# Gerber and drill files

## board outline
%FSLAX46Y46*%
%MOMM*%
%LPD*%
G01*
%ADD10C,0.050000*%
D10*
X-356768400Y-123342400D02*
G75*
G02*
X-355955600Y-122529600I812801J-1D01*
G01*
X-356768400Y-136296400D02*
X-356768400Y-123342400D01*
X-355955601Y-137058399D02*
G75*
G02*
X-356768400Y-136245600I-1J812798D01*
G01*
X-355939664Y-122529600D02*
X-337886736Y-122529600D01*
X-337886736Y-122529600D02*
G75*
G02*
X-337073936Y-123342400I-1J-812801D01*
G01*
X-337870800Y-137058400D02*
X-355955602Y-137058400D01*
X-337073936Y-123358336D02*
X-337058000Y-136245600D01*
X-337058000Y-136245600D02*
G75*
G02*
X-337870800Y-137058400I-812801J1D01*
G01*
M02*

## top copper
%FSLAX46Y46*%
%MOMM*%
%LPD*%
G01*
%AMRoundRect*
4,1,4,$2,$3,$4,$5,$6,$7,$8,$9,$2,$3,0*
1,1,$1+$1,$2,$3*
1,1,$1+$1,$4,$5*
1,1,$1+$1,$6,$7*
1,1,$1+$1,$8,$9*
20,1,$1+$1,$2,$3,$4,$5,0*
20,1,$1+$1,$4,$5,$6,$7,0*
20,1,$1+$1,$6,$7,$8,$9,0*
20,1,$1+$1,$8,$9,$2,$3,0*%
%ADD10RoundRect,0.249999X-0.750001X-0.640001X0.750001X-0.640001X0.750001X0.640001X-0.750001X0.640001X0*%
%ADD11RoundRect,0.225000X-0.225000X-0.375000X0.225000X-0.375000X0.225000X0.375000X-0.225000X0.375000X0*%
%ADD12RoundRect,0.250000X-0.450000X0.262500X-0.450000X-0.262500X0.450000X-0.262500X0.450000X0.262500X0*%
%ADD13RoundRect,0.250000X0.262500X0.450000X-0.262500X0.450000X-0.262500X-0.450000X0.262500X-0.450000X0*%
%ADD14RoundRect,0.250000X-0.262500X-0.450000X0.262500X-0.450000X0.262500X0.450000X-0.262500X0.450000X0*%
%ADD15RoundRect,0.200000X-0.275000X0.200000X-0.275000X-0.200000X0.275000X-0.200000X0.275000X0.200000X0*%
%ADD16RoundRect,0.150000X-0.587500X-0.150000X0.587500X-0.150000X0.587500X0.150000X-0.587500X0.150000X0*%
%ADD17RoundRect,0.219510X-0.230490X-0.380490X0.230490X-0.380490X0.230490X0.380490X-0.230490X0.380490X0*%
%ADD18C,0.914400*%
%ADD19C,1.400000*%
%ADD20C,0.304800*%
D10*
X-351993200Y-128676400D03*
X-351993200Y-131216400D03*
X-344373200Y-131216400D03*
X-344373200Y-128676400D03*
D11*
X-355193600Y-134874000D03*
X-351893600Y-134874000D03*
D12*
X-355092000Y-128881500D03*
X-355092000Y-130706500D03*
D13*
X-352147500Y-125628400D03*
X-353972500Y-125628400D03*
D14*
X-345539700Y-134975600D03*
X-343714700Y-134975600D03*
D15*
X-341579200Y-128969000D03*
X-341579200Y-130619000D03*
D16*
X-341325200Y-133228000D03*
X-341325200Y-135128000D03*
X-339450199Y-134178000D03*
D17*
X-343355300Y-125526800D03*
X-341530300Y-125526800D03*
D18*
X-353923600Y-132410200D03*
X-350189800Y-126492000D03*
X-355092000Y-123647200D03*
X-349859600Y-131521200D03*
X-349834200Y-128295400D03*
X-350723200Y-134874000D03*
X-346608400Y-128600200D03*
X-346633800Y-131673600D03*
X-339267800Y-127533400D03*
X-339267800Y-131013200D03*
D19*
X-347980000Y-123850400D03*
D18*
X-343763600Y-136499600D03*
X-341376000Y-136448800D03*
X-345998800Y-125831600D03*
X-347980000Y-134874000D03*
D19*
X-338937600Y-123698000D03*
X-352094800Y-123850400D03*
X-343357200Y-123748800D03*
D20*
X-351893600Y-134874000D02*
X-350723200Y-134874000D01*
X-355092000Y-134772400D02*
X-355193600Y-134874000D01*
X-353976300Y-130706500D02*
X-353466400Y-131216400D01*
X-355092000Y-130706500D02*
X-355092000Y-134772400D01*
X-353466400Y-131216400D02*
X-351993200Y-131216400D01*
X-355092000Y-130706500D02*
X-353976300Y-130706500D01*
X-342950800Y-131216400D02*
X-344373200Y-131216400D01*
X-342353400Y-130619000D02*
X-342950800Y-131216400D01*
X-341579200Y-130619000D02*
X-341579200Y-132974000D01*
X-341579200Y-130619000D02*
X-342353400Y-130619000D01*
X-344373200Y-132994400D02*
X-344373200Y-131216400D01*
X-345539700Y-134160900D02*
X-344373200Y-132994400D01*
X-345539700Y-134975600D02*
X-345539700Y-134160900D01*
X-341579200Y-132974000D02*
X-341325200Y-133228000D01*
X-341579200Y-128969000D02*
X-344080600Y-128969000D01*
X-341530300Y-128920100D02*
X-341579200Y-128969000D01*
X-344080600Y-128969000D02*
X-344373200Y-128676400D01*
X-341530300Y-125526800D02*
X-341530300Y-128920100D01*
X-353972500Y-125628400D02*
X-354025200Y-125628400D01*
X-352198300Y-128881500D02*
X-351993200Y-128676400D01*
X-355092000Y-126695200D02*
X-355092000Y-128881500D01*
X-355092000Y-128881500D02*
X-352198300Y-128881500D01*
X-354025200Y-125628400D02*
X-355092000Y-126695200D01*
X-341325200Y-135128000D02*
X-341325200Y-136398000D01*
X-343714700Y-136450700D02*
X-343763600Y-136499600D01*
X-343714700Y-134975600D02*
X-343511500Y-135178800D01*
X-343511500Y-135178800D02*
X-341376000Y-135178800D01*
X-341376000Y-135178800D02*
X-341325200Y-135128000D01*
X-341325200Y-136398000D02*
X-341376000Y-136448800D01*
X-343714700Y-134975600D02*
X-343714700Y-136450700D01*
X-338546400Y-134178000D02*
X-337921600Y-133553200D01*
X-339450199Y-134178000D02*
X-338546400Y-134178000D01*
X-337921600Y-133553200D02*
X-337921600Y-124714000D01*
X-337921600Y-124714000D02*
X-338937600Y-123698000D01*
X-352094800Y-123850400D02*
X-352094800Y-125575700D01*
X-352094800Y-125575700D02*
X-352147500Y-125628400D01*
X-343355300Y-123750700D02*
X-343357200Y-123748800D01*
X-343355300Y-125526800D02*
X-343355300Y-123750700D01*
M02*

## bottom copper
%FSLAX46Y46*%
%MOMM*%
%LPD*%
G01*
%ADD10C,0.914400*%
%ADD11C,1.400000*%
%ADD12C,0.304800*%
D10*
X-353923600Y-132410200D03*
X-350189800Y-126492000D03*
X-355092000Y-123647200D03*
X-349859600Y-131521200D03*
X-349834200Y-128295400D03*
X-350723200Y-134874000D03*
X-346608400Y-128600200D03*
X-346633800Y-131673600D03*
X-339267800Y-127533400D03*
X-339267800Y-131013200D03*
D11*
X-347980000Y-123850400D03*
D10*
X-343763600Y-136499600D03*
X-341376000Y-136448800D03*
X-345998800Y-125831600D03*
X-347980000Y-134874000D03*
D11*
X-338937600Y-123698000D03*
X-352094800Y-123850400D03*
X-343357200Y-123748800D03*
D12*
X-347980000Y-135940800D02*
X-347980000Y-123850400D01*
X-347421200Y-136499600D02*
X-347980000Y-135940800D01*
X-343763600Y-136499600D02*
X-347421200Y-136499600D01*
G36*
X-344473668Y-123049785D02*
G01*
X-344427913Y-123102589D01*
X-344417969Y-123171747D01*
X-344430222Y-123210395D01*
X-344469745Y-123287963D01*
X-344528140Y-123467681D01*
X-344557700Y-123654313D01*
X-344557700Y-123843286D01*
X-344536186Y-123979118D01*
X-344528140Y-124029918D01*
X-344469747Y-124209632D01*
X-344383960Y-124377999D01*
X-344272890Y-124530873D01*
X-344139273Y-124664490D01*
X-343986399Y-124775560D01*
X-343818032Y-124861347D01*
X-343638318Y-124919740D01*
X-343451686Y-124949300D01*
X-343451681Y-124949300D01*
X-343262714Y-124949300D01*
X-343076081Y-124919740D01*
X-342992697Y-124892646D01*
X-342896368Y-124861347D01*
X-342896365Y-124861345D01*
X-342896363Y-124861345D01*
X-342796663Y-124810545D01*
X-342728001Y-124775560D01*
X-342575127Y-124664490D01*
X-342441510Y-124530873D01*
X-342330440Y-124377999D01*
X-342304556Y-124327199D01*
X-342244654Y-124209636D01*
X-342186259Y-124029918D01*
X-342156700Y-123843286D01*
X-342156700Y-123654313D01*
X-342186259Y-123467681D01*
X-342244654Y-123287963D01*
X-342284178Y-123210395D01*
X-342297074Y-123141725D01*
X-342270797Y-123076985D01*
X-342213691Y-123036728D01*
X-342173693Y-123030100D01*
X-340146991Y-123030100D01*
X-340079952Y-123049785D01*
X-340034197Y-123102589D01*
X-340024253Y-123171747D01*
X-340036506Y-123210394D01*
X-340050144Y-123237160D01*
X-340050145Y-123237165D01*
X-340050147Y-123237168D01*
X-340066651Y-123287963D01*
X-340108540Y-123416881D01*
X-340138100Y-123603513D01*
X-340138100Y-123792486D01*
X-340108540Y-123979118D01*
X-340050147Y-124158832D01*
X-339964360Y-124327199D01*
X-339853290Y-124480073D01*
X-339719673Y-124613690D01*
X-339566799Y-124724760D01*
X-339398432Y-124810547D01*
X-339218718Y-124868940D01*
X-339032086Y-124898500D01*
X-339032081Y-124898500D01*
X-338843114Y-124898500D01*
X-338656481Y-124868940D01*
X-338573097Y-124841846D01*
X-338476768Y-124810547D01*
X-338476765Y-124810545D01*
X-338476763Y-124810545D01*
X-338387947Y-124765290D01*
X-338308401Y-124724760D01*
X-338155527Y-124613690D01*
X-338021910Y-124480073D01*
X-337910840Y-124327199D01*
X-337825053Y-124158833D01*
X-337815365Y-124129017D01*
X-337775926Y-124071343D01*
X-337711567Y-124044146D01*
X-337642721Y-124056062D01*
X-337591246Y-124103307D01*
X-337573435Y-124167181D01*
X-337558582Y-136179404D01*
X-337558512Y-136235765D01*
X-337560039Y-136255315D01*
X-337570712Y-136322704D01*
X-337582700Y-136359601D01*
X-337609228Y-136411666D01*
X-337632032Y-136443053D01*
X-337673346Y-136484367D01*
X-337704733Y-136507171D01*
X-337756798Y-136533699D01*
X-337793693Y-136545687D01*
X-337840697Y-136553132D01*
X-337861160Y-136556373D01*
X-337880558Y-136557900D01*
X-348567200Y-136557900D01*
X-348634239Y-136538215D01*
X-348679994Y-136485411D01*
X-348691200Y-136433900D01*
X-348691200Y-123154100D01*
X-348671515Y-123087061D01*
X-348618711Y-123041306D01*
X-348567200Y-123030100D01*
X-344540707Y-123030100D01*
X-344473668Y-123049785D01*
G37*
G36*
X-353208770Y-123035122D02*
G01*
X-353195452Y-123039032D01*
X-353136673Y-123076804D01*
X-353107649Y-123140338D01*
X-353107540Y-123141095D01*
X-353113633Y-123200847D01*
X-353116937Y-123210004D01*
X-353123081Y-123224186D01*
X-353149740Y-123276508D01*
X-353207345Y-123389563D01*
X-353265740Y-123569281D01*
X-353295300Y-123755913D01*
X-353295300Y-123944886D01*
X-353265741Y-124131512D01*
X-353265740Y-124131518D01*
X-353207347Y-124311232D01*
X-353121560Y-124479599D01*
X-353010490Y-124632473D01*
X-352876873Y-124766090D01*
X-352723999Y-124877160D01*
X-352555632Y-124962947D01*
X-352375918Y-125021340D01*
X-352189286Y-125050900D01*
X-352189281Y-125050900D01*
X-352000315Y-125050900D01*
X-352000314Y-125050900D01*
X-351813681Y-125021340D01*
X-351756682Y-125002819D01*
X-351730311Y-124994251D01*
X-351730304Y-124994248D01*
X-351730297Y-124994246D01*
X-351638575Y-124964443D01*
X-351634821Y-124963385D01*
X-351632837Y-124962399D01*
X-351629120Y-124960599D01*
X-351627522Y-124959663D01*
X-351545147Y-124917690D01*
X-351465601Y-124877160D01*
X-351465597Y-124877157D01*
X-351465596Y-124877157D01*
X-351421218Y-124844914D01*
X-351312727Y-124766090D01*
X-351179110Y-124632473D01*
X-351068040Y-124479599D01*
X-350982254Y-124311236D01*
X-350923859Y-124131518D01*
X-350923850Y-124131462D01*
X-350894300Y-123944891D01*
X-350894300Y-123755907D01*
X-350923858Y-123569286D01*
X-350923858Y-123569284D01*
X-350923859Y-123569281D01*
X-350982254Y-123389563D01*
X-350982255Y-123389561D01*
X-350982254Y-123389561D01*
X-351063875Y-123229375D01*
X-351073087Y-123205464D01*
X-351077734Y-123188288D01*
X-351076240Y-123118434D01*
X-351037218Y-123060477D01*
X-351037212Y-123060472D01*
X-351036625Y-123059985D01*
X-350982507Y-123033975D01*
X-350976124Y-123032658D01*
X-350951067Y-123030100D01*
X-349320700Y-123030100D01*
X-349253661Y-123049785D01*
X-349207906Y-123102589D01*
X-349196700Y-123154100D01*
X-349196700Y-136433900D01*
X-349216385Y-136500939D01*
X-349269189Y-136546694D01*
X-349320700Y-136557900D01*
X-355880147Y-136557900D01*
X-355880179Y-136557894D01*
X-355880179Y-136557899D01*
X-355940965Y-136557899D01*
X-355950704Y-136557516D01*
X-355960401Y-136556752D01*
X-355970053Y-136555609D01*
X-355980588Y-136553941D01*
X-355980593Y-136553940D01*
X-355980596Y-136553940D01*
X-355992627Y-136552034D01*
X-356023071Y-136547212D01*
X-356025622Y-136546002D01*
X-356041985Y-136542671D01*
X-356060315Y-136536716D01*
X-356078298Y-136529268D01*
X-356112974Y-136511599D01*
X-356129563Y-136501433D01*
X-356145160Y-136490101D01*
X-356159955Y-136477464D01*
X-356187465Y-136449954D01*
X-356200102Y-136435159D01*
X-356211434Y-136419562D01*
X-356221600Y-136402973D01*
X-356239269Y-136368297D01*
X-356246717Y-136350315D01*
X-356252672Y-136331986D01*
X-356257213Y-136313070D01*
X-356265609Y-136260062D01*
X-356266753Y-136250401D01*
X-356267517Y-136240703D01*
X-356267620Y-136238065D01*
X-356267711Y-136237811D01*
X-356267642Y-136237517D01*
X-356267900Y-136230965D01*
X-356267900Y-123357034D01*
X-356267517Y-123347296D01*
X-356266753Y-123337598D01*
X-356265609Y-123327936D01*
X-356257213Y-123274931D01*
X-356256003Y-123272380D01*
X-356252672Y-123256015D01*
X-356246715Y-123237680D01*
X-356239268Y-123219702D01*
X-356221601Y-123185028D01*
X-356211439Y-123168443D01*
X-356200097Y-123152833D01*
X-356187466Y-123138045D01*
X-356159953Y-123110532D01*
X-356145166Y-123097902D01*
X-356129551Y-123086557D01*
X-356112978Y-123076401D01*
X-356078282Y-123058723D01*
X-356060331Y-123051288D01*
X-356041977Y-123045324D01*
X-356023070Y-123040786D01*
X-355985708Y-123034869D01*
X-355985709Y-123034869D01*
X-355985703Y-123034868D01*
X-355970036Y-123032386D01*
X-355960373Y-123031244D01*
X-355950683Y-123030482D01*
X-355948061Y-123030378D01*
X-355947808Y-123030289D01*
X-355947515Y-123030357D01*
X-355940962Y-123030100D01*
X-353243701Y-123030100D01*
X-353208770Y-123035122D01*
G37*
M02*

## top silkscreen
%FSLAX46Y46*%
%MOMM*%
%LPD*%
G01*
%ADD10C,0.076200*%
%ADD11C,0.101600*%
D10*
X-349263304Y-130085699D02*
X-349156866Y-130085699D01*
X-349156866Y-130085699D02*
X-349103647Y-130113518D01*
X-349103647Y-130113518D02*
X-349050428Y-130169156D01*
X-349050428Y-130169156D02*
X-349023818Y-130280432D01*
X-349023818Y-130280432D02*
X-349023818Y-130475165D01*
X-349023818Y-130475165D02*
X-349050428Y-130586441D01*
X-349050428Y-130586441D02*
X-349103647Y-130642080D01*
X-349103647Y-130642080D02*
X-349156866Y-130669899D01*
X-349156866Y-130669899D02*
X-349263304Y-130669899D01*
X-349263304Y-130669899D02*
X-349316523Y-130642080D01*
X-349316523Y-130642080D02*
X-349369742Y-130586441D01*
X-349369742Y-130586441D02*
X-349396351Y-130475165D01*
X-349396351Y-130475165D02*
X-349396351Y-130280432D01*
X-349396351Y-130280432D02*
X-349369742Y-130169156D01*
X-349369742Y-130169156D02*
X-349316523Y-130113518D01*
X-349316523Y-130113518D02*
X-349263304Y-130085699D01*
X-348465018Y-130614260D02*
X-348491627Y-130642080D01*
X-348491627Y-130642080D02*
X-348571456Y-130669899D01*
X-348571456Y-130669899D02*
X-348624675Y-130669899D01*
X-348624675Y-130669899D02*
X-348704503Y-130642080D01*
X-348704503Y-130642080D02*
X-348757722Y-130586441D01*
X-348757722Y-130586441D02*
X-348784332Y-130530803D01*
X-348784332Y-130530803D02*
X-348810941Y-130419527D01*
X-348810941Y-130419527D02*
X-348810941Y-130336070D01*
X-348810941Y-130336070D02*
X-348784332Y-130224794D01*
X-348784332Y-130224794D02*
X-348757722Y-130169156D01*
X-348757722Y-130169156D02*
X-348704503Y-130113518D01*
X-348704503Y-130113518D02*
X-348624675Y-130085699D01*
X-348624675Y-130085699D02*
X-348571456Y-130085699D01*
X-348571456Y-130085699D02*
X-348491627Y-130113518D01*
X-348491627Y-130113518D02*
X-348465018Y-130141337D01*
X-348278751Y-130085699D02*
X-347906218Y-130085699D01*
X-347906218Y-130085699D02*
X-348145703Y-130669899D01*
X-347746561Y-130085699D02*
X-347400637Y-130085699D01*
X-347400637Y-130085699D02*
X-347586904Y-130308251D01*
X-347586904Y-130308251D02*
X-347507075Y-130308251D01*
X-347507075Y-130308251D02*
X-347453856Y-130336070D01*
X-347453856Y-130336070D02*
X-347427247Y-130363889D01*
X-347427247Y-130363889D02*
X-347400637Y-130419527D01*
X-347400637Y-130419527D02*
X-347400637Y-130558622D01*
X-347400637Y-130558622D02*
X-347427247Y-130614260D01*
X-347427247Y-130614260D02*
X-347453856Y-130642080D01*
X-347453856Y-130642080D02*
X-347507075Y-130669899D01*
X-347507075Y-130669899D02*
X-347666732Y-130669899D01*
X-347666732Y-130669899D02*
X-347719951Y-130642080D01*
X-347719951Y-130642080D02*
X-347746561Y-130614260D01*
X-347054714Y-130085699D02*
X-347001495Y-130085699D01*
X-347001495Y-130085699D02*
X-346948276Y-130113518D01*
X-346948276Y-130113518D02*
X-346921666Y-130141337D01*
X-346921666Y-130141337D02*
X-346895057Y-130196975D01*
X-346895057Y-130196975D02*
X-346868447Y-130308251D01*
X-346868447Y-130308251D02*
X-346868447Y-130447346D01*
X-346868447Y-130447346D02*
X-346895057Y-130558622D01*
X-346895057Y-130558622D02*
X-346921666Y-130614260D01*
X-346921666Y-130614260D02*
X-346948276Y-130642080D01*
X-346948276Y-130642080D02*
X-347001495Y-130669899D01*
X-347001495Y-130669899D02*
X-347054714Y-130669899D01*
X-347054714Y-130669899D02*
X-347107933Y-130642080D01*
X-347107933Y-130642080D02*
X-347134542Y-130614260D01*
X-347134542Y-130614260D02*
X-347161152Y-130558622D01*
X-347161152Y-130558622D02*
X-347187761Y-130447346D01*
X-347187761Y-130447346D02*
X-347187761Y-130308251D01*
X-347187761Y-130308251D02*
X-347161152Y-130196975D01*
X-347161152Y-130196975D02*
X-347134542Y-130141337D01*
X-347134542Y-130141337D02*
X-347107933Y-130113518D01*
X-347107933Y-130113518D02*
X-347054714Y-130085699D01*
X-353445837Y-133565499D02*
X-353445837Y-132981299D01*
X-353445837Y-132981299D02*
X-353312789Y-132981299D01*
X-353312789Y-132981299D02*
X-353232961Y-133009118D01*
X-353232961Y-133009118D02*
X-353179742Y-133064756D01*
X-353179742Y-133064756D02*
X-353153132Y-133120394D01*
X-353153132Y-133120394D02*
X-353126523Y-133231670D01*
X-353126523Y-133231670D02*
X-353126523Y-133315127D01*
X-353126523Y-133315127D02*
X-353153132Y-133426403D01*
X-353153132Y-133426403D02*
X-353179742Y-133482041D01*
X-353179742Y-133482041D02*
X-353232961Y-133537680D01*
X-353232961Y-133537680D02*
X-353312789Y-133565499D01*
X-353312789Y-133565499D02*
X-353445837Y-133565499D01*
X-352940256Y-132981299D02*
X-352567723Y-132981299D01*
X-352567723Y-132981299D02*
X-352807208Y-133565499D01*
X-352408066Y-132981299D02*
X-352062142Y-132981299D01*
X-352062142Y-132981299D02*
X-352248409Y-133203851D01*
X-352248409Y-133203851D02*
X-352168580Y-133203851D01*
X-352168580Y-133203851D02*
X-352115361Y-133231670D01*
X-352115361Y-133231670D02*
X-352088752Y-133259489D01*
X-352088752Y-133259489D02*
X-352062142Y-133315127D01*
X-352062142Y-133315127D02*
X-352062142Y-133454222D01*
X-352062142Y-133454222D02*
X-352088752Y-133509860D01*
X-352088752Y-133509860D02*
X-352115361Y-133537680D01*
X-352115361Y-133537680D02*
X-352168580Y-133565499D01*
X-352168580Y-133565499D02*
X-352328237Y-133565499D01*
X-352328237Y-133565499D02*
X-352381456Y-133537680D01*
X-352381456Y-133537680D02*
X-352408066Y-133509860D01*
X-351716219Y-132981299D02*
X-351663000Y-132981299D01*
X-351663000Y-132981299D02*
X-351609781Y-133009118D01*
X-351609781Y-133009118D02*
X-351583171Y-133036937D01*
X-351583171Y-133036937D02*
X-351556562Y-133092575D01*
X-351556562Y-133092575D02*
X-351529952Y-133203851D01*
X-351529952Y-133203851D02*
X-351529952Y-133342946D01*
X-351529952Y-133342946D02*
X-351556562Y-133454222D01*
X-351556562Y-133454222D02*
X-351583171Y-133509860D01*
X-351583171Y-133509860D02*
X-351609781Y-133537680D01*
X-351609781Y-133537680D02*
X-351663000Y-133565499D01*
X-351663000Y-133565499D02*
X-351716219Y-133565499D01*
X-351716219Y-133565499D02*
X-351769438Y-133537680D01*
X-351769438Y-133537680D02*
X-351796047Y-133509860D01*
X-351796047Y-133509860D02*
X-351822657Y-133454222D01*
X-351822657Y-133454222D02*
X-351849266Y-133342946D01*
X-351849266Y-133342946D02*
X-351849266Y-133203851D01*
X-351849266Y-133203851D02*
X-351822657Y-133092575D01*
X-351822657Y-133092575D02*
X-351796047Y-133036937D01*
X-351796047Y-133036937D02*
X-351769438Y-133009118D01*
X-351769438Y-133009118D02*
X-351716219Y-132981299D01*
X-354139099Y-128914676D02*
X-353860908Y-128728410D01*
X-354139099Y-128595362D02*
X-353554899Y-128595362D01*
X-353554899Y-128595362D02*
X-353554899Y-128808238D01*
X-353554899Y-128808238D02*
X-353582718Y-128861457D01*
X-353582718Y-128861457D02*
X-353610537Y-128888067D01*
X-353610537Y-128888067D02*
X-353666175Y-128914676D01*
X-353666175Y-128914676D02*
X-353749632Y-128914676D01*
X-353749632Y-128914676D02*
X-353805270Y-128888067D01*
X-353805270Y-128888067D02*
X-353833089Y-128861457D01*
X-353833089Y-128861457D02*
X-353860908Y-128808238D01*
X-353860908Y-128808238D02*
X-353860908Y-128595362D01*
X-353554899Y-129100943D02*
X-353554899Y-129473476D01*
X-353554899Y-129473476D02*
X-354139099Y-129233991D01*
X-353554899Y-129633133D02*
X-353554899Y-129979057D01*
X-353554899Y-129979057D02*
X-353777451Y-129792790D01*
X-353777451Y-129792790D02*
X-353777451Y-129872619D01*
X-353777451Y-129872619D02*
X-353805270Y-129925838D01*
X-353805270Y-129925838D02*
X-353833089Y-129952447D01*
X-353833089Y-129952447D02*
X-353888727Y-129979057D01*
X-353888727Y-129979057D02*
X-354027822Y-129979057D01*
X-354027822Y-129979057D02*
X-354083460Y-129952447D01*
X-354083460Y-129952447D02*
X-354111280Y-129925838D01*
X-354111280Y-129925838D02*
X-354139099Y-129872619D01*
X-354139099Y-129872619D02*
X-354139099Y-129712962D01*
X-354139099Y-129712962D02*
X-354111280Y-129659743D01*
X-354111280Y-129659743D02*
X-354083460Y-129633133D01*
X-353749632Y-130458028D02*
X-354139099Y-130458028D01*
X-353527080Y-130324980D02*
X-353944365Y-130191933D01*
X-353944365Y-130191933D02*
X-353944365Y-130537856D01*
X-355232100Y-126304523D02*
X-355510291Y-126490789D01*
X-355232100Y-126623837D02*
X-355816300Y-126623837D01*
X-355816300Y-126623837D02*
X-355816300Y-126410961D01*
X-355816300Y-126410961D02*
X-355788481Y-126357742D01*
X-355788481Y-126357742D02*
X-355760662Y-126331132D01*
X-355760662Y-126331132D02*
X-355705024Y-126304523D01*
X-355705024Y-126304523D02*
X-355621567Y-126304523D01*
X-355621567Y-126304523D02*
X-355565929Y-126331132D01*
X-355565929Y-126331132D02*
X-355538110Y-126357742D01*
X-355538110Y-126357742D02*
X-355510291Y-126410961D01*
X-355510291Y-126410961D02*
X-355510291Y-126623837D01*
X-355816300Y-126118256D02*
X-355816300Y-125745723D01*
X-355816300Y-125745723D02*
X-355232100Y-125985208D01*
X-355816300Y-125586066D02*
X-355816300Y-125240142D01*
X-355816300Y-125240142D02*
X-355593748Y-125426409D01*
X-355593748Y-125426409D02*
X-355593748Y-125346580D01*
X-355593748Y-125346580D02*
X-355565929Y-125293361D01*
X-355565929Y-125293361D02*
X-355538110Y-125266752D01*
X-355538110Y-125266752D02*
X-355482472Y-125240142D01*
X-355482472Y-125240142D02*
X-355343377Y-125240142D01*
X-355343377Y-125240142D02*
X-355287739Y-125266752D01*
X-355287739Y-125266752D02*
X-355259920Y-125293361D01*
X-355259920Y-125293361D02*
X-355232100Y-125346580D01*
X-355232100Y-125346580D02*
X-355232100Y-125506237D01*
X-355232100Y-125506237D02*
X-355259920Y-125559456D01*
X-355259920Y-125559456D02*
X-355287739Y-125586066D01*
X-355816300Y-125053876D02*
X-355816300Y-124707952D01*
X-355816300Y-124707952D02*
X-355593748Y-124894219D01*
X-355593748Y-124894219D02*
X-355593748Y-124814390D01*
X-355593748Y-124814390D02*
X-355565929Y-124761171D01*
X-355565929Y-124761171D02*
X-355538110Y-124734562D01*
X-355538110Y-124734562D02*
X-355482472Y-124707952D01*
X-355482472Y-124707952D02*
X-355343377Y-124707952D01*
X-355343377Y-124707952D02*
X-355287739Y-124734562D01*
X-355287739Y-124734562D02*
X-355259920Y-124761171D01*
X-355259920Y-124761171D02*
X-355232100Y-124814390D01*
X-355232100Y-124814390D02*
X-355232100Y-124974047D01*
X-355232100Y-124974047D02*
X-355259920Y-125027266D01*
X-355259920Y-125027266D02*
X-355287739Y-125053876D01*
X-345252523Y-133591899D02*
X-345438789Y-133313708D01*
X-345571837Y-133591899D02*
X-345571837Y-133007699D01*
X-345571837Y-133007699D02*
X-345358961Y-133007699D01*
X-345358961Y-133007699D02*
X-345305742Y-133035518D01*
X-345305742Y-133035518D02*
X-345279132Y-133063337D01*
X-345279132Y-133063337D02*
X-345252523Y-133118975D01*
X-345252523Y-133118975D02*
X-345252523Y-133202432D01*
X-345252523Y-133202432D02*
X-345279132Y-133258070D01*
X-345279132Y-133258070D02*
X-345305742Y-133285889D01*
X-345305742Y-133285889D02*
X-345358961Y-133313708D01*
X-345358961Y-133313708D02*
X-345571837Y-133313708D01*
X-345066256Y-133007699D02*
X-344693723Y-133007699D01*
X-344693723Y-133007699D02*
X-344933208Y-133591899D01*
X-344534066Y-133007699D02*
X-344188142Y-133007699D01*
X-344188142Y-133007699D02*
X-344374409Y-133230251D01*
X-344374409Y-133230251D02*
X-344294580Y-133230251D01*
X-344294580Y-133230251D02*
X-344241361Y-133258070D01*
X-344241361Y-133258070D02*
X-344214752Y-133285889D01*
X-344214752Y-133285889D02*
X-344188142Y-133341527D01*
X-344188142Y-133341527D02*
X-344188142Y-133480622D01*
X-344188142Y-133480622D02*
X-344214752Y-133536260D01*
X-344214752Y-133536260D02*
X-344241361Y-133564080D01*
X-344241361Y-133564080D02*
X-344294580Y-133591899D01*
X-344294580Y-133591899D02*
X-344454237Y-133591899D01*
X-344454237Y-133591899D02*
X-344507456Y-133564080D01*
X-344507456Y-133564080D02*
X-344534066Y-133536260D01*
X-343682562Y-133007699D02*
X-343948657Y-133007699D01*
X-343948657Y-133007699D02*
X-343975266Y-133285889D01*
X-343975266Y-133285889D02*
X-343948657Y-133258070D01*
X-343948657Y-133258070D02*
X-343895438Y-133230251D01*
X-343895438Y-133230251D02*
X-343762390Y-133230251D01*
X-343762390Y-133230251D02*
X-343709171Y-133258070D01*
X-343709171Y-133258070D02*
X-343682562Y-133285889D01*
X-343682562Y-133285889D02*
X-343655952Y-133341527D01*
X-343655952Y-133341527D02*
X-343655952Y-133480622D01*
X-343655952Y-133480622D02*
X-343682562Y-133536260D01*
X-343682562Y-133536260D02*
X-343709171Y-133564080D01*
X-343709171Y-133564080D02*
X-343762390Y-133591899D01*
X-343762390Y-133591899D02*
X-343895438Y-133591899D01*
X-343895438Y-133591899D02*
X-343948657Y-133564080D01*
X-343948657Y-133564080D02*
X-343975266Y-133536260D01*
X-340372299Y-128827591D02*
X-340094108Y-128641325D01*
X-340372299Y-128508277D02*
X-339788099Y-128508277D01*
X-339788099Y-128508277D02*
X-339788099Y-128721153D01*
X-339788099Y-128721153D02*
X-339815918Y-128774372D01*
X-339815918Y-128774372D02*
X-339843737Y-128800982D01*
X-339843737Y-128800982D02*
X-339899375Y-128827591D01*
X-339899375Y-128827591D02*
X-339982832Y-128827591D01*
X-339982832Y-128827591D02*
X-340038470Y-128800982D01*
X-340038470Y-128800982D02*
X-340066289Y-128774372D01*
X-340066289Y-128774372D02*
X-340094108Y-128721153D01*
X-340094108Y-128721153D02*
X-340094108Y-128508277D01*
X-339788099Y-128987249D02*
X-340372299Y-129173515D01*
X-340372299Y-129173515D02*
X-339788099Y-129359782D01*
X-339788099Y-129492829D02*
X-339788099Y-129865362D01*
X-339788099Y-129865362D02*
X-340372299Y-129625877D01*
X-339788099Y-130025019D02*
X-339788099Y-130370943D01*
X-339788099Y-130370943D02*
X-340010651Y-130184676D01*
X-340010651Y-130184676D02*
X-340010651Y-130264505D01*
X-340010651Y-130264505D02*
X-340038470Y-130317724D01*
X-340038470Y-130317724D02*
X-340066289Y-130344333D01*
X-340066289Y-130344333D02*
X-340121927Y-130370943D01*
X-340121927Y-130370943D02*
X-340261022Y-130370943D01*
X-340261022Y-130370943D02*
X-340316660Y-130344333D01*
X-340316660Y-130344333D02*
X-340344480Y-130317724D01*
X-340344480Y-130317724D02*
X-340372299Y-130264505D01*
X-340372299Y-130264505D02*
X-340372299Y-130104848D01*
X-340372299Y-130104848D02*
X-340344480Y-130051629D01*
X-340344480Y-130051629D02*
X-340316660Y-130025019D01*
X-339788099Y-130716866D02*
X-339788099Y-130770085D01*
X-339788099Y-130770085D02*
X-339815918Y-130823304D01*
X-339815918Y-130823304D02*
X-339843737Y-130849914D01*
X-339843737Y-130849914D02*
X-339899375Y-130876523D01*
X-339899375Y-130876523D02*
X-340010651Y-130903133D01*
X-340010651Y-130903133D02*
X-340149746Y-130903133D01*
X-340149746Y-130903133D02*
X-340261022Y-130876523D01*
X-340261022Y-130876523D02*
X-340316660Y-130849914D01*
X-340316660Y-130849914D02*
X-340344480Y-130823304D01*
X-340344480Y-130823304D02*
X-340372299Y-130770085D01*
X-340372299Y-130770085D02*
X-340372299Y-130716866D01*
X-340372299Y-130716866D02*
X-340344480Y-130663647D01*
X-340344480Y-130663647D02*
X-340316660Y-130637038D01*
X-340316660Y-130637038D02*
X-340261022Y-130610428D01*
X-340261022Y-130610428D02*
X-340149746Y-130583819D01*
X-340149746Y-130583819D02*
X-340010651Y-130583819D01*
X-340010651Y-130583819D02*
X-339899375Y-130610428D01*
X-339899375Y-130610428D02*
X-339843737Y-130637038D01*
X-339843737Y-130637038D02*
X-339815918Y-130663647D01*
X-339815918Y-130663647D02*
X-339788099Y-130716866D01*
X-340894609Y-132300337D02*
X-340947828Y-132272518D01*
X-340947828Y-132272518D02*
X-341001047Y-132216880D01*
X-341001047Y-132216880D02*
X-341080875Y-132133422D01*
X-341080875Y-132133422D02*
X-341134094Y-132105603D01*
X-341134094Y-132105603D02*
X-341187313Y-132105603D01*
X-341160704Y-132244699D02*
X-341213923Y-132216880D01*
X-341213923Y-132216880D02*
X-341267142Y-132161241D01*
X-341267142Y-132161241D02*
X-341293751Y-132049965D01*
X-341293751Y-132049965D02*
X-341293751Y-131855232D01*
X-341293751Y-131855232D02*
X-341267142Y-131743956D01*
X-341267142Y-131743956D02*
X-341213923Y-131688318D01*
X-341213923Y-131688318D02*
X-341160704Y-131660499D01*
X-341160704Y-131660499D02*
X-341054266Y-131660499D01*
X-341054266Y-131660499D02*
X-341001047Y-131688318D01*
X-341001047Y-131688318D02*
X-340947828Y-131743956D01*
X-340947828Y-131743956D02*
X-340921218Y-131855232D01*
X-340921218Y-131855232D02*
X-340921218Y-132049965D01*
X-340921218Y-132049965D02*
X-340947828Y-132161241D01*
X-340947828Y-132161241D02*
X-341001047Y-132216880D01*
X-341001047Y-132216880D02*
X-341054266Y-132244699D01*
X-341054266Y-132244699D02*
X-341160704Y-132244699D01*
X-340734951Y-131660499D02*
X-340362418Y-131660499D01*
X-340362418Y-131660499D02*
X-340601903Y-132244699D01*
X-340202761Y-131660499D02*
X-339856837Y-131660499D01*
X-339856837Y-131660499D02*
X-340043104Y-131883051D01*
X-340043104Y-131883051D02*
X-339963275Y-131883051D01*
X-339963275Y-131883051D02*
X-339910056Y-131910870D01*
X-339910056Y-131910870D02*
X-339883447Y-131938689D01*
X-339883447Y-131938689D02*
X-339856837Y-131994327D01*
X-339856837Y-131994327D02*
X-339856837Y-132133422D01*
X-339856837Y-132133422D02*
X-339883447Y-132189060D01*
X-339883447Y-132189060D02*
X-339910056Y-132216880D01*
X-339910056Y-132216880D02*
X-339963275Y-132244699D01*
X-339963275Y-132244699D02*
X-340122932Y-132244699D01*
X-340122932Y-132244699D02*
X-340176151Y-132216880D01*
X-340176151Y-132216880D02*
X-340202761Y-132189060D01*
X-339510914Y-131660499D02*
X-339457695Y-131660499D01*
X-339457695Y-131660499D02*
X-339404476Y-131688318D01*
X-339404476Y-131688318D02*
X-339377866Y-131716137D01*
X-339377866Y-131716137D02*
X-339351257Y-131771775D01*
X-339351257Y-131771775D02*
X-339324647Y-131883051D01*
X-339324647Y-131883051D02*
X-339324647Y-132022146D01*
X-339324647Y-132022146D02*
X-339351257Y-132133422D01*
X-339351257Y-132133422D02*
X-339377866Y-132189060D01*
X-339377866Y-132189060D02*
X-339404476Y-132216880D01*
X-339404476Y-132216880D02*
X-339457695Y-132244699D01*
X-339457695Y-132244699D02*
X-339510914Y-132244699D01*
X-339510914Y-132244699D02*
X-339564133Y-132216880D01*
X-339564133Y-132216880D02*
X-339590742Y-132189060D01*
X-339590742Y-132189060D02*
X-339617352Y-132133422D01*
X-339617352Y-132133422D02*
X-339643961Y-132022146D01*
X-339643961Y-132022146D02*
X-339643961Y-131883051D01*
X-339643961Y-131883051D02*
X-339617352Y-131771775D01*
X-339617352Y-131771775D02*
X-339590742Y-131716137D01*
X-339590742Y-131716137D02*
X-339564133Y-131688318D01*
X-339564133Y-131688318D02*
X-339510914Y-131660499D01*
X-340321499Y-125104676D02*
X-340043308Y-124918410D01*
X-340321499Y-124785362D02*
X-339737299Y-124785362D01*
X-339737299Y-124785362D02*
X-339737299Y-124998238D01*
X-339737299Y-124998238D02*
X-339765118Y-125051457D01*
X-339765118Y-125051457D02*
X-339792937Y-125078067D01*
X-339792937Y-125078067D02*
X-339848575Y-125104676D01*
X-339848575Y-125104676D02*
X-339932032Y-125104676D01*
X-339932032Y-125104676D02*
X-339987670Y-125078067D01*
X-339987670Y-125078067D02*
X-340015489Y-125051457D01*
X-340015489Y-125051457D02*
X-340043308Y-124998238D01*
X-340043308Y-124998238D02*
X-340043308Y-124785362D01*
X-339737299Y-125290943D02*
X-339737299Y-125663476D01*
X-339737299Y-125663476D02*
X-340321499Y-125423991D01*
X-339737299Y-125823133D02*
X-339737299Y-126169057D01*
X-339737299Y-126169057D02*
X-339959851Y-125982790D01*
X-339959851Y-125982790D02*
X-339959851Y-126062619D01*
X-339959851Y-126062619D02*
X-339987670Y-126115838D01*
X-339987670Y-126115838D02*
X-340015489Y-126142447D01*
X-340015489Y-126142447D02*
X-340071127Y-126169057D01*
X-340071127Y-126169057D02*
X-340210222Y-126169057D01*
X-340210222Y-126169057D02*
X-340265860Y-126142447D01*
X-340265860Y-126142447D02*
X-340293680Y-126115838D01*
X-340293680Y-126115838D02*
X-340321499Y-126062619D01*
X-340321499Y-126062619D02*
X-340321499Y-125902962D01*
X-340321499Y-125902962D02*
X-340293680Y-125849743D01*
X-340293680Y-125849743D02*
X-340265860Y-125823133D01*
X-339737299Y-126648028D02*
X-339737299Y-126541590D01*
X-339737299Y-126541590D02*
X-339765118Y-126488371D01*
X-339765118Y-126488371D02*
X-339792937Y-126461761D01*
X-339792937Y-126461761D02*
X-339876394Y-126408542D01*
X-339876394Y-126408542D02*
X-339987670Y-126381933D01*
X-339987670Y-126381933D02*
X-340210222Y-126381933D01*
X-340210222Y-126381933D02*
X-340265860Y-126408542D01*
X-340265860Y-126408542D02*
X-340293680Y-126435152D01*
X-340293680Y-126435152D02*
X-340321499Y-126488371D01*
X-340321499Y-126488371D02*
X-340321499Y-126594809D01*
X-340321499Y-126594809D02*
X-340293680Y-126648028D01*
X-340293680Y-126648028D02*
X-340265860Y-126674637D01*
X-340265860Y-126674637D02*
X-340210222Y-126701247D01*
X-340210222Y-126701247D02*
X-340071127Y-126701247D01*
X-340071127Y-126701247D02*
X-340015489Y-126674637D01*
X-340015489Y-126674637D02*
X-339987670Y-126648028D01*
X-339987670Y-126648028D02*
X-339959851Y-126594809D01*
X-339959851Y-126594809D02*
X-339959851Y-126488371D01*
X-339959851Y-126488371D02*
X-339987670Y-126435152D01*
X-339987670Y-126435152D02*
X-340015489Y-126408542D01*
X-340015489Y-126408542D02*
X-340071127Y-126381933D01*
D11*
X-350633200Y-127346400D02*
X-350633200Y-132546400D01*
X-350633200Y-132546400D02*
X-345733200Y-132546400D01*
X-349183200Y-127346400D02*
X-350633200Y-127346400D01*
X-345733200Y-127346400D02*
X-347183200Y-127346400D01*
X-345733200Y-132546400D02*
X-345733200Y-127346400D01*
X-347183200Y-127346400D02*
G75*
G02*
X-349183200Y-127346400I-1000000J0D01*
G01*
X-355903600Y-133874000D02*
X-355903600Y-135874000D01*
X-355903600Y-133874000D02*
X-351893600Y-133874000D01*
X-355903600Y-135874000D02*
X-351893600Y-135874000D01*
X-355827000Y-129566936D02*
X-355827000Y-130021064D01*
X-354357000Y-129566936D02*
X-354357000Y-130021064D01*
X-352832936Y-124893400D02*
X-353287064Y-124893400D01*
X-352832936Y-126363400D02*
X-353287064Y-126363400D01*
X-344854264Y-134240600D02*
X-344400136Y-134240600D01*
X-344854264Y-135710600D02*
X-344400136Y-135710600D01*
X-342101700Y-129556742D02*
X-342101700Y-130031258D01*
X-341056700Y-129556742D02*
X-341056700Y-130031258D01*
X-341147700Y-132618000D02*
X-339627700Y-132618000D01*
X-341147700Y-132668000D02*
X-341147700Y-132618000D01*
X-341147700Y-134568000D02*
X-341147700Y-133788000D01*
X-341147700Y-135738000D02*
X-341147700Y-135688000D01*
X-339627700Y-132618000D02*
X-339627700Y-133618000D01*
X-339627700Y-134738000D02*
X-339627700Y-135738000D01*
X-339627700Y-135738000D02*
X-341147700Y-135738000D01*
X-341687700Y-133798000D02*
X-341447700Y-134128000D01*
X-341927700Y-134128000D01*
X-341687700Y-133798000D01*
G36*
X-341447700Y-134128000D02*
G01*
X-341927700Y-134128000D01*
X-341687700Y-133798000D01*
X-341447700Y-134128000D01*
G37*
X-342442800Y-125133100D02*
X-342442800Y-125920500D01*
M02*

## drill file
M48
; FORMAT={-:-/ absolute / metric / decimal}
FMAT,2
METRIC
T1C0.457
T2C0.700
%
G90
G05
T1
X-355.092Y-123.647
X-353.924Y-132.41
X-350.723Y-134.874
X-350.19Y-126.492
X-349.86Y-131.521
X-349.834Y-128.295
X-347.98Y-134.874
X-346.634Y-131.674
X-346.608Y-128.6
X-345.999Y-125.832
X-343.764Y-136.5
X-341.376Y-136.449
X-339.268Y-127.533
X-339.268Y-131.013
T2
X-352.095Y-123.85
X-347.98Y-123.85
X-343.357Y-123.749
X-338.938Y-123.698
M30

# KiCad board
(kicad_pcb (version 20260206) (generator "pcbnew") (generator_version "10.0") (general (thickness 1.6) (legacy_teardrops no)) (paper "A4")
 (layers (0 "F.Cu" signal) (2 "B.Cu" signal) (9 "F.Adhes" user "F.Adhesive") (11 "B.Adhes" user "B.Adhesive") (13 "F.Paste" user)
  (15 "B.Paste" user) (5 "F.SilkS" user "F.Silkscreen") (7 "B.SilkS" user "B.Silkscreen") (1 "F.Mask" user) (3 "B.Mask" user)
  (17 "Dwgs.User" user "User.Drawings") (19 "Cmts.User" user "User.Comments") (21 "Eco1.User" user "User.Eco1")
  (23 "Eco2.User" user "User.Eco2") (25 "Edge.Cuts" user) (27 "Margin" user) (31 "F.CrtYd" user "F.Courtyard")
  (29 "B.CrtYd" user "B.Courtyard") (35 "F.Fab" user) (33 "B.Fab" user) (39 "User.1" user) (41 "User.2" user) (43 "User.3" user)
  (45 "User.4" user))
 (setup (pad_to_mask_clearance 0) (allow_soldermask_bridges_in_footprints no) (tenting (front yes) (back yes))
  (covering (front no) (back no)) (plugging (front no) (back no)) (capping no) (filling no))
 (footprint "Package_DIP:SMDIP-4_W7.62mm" (layer "F.Cu") (at -348.1832 129.9464)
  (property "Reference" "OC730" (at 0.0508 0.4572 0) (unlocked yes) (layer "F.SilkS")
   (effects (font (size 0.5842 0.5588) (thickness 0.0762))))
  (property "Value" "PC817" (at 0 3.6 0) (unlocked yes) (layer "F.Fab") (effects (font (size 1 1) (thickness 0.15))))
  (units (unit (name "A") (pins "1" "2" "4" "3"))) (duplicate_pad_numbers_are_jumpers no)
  (fp_line (start -2.45 -2.6) (end -2.45 2.6) (stroke (width 0.1016) (type solid)) (layer "F.SilkS"))
  (fp_line (start -2.45 2.6) (end 2.45 2.6) (stroke (width 0.1016) (type solid)) (layer "F.SilkS"))
  (fp_line (start -1 -2.6) (end -2.45 -2.6) (stroke (width 0.1016) (type solid)) (layer "F.SilkS"))
  (fp_line (start 2.45 -2.6) (end 1 -2.6) (stroke (width 0.1016) (type solid)) (layer "F.SilkS"))
  (fp_line (start 2.45 2.6) (end 2.45 -2.6) (stroke (width 0.1016) (type solid)) (layer "F.SilkS"))
  (fp_arc (start 1 -2.6) (mid 0 -1.6) (end -1 -2.6) (stroke (width 0.1016) (type solid)) (layer "F.SilkS"))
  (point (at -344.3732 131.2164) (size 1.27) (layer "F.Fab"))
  (pad "1" smd roundrect (at -3.81 -1.27) (size 2 1.78) (layers "F.Cu" "F.Mask" "F.Paste") (roundrect_rratio 0.140449)
   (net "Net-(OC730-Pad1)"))
  (pad "2" smd roundrect (at -3.81 1.27) (size 2 1.78) (layers "F.Cu" "F.Mask" "F.Paste") (roundrect_rratio 0.140449) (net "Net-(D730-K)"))
  (pad "3" smd roundrect (at 3.81 1.27) (size 2 1.78) (layers "F.Cu" "F.Mask" "F.Paste") (roundrect_rratio 0.140449) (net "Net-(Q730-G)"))
  (pad "4" smd roundrect (at 3.81 -1.27) (size 2 1.78) (layers "F.Cu" "F.Mask" "F.Paste") (roundrect_rratio 0.140449)
   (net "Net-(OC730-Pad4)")))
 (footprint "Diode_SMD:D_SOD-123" (layer "F.Cu") (at -353.5436 134.874)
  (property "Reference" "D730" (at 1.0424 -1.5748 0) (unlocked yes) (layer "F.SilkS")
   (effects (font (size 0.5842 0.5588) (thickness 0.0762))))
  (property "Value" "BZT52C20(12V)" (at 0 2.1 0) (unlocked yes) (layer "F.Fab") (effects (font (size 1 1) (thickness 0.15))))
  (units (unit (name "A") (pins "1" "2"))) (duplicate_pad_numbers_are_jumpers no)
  (fp_line (start -2.36 -1) (end -2.36 1) (stroke (width 0.1016) (type solid)) (layer "F.SilkS"))
  (fp_line (start -2.36 -1) (end 1.65 -1) (stroke (width 0.1016) (type solid)) (layer "F.SilkS"))
  (fp_line (start -2.36 1) (end 1.65 1) (stroke (width 0.1016) (type solid)) (layer "F.SilkS"))
  (pad "1" smd roundrect (at -1.65 0) (size 0.9 1.2) (layers "F.Cu" "F.Mask" "F.Paste") (roundrect_rratio 0.25) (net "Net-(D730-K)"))
  (pad "2" smd roundrect (at 1.65 0) (size 0.9 1.2) (layers "F.Cu" "F.Mask" "F.Paste") (roundrect_rratio 0.25) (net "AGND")))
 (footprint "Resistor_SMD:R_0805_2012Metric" (layer "F.Cu") (at -355.092 129.794 -90)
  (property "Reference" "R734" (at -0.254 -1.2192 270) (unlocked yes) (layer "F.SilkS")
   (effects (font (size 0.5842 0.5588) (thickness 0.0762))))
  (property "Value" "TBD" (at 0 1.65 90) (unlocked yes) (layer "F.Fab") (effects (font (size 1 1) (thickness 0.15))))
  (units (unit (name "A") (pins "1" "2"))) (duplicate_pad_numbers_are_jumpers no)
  (fp_line (start -0.227064 0.735) (end 0.227064 0.735) (stroke (width 0.1016) (type solid)) (layer "F.SilkS"))
  (fp_line (start -0.227064 -0.735) (end 0.227064 -0.735) (stroke (width 0.1016) (type solid)) (layer "F.SilkS"))
  (pad "1" smd roundrect (at -0.9125 0 270) (size 1.025 1.4) (layers "F.Cu" "F.Mask" "F.Paste") (roundrect_rratio 0.243902)
   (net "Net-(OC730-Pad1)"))
  (pad "2" smd roundrect (at 0.9125 0 270) (size 1.025 1.4) (layers "F.Cu" "F.Mask" "F.Paste") (roundrect_rratio 0.243902)
   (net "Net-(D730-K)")))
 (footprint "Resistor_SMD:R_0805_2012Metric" (layer "F.Cu") (at -353.06 125.6284 180)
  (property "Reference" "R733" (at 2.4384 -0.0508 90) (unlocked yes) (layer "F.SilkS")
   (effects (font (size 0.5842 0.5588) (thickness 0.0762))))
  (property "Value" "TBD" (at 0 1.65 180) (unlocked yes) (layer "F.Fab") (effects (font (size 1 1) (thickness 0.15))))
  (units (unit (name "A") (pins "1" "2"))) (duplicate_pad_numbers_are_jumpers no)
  (fp_line (start -0.227064 0.735) (end 0.227064 0.735) (stroke (width 0.1016) (type solid)) (layer "F.SilkS"))
  (fp_line (start -0.227064 -0.735) (end 0.227064 -0.735) (stroke (width 0.1016) (type solid)) (layer "F.SilkS"))
  (pad "1" smd roundrect (at -0.9125 0 180) (size 1.025 1.4) (layers "F.Cu" "F.Mask" "F.Paste") (roundrect_rratio 0.243902) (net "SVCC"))
  (pad "2" smd roundrect (at 0.9125 0 180) (size 1.025 1.4) (layers "F.Cu" "F.Mask" "F.Paste") (roundrect_rratio 0.243902)
   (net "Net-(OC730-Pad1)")))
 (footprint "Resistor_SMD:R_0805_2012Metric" (layer "F.Cu") (at -344.6272 134.9756)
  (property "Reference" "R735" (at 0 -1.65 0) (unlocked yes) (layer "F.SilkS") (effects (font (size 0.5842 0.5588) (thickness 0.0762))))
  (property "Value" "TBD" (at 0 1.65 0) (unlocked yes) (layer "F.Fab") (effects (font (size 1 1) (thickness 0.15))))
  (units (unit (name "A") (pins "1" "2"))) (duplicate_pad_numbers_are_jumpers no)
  (fp_line (start -0.227064 -0.735) (end 0.227064 -0.735) (stroke (width 0.1016) (type solid)) (layer "F.SilkS"))
  (fp_line (start -0.227064 0.735) (end 0.227064 0.735) (stroke (width 0.1016) (type solid)) (layer "F.SilkS"))
  (pad "1" smd roundrect (at -0.9125 0) (size 1.025 1.4) (layers "F.Cu" "F.Mask" "F.Paste") (roundrect_rratio 0.243902) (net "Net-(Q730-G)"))
  (pad "2" smd roundrect (at 0.9125 0) (size 1.025 1.4) (layers "F.Cu" "F.Mask" "F.Paste") (roundrect_rratio 0.243902) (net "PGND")))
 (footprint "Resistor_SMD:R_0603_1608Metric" (layer "F.Cu") (at -341.5792 129.794 -90)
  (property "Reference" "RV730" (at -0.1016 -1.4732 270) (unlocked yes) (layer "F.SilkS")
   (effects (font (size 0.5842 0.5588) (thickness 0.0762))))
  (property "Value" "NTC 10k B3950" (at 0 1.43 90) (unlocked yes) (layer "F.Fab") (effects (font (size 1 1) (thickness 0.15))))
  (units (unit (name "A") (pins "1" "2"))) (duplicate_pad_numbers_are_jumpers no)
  (fp_line (start -0.237258 0.5225) (end 0.237258 0.5225) (stroke (width 0.1016) (type solid)) (layer "F.SilkS"))
  (fp_line (start -0.237258 -0.5225) (end 0.237258 -0.5225) (stroke (width 0.1016) (type solid)) (layer "F.SilkS"))
  (pad "1" smd roundrect (at -0.825 0 270) (size 0.8 0.95) (layers "F.Cu" "F.Mask" "F.Paste") (roundrect_rratio 0.25)
   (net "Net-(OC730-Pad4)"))
  (pad "2" smd roundrect (at 0.825 0 270) (size 0.8 0.95) (layers "F.Cu" "F.Mask" "F.Paste") (roundrect_rratio 0.25) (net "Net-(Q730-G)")))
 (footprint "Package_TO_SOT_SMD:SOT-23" (layer "F.Cu") (at -340.3877 134.178)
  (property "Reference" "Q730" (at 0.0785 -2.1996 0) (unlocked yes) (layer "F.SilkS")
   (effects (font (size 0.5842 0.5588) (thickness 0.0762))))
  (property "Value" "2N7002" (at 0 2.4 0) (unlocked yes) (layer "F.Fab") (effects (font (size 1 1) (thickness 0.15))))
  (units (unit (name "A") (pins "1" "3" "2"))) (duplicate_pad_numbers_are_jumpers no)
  (fp_line (start -0.76 -1.56) (end 0.76 -1.56) (stroke (width 0.1016) (type solid)) (layer "F.SilkS"))
  (fp_line (start -0.76 -1.51) (end -0.76 -1.56) (stroke (width 0.1016) (type solid)) (layer "F.SilkS"))
  (fp_line (start -0.76 0.39) (end -0.76 -0.39) (stroke (width 0.1016) (type solid)) (layer "F.SilkS"))
  (fp_line (start -0.76 1.56) (end -0.76 1.51) (stroke (width 0.1016) (type solid)) (layer "F.SilkS"))
  (fp_line (start 0.76 -1.56) (end 0.76 -0.56) (stroke (width 0.1016) (type solid)) (layer "F.SilkS"))
  (fp_line (start 0.76 0.56) (end 0.76 1.56) (stroke (width 0.1016) (type solid)) (layer "F.SilkS"))
  (fp_line (start 0.76 1.56) (end -0.76 1.56) (stroke (width 0.1016) (type solid)) (layer "F.SilkS"))
  (fp_poly (pts (xy -1.3 -0.38) (xy -1.06 -0.05) (xy -1.54 -0.05)) (stroke (width 0.1016) (type solid)) (fill yes) (layer "F.SilkS"))
  (pad "1" smd roundrect (at -0.9375 -0.95) (size 1.475 0.6) (layers "F.Cu" "F.Mask" "F.Paste") (roundrect_rratio 0.25) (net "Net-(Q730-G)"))
  (pad "2" smd roundrect (at -0.9375 0.95) (size 1.475 0.6) (layers "F.Cu" "F.Mask" "F.Paste") (roundrect_rratio 0.25) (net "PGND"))
  (pad "3" smd roundrect (at 0.937501 0) (size 1.475 0.6) (layers "F.Cu" "F.Mask" "F.Paste") (roundrect_rratio 0.25) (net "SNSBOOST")))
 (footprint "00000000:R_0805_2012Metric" (layer "F.Cu") (at -342.4428 125.5268)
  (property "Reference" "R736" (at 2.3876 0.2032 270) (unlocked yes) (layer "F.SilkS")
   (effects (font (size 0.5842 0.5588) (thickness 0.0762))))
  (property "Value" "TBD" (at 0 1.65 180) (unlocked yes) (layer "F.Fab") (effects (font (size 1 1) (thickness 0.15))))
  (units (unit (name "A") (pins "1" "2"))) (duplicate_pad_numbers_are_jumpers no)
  (fp_line (start 0 -0.3937) (end 0 0.3937) (stroke (width 0.1016) (type default)) (layer "F.SilkS"))
  (pad "1" smd roundrect (at -0.9125 0) (size 0.9 1.2) (layers "F.Cu" "F.Mask" "F.Paste") (roundrect_rratio 0.2439004878) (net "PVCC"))
  (pad "2" smd roundrect (at 0.9125 0) (size 0.9 1.2) (layers "F.Cu" "F.Mask" "F.Paste") (roundrect_rratio 0.2439004878)
   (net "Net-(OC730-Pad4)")))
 (gr_arc (start -356.7684 123.3424) (mid -356.530336 122.767664) (end -355.9556 122.5296) (stroke (width 0.05) (type default))
  (layer "Edge.Cuts"))
 (gr_line (start -356.7684 136.2964) (end -356.7684 123.3424) (stroke (width 0.05) (type default)) (layer "Edge.Cuts"))
 (gr_arc (start -355.955601 137.058399) (mid -356.530337 136.820336) (end -356.7684 136.2456) (stroke (width 0.05) (type default))
  (layer "Edge.Cuts"))
 (gr_line (start -355.939664 122.5296) (end -337.886736 122.5296) (stroke (width 0.05) (type default)) (layer "Edge.Cuts"))
 (gr_arc (start -337.886736 122.5296) (mid -337.312 122.767664) (end -337.073936 123.3424) (stroke (width 0.05) (type default))
  (layer "Edge.Cuts"))
 (gr_line (start -337.8708 137.0584) (end -355.955602 137.0584) (stroke (width 0.05) (type default)) (layer "Edge.Cuts"))
 (gr_line (start -337.073936 123.358336) (end -337.058 136.2456) (stroke (width 0.05) (type default)) (layer "Edge.Cuts"))
 (gr_arc (start -337.058 136.2456) (mid -337.296064 136.820336) (end -337.8708 137.0584) (stroke (width 0.05) (type default))
  (layer "Edge.Cuts"))
 (segment (start -351.8936 134.874) (end -350.7232 134.874) (width 0.3048) (layer "F.Cu") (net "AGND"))
 (via (at -353.9236 132.4102) (size 0.9144) (drill 0.4572) (layers "F.Cu" "B.Cu") (tenting (front no) (back no)) (capping no)
  (covering (front no) (back no)) (plugging (front no) (back no)) (filling no) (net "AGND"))
 (via (at -350.1898 126.492) (size 0.9144) (drill 0.4572) (layers "F.Cu" "B.Cu") (tenting (front no) (back no)) (capping no)
  (covering (front no) (back no)) (plugging (front no) (back no)) (filling no) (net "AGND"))
 (via (at -355.092 123.6472) (size 0.9144) (drill 0.4572) (layers "F.Cu" "B.Cu") (tenting (front no) (back no)) (capping no)
  (covering (front no) (back no)) (plugging (front no) (back no)) (filling no) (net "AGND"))
 (via (at -349.8596 131.5212) (size 0.9144) (drill 0.4572) (layers "F.Cu" "B.Cu") (tenting (front no) (back no)) (capping no)
  (covering (front no) (back no)) (plugging (front no) (back no)) (filling no) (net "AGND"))
 (via (at -349.8342 128.2954) (size 0.9144) (drill 0.4572) (layers "F.Cu" "B.Cu") (tenting (front no) (back no)) (capping no)
  (covering (front no) (back no)) (plugging (front no) (back no)) (filling no) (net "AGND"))
 (via (at -350.7232 134.874) (size 0.9144) (drill 0.4572) (layers "F.Cu" "B.Cu") (tenting (front no) (back no)) (capping no)
  (covering (front no) (back no)) (plugging (front no) (back no)) (filling no) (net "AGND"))
 (segment (start -355.092 134.7724) (end -355.1936 134.874) (width 0.3048) (layer "F.Cu") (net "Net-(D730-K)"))
 (segment (start -353.9763 130.7065) (end -353.4664 131.2164) (width 0.3048) (layer "F.Cu") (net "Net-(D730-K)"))
 (segment (start -355.092 130.7065) (end -355.092 134.7724) (width 0.3048) (layer "F.Cu") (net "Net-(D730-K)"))
 (segment (start -353.4664 131.2164) (end -351.9932 131.2164) (width 0.3048) (layer "F.Cu") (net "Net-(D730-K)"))
 (segment (start -355.092 130.7065) (end -353.9763 130.7065) (width 0.3048) (layer "F.Cu") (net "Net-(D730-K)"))
 (segment (start -342.9508 131.2164) (end -344.3732 131.2164) (width 0.3048) (layer "F.Cu") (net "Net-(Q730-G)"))
 (segment (start -342.3534 130.619) (end -342.9508 131.2164) (width 0.3048) (layer "F.Cu") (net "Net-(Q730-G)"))
 (segment (start -341.5792 130.619) (end -341.5792 132.974) (width 0.3048) (layer "F.Cu") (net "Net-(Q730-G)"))
 (segment (start -341.5792 130.619) (end -342.3534 130.619) (width 0.3048) (layer "F.Cu") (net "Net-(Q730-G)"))
 (segment (start -344.3732 132.9944) (end -344.3732 131.2164) (width 0.3048) (layer "F.Cu") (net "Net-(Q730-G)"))
 (segment (start -345.5397 134.1609) (end -344.3732 132.9944) (width 0.3048) (layer "F.Cu") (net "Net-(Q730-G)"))
 (segment (start -345.5397 134.9756) (end -345.5397 134.1609) (width 0.3048) (layer "F.Cu") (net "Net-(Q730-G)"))
 (segment (start -341.5792 132.974) (end -341.3252 133.228) (width 0.3048) (layer "F.Cu") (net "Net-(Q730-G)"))
 (segment (start -341.5792 128.969) (end -344.0806 128.969) (width 0.3048) (layer "F.Cu") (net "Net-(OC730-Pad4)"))
 (segment (start -341.5303 128.9201) (end -341.5792 128.969) (width 0.3048) (layer "F.Cu") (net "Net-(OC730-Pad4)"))
 (segment (start -344.0806 128.969) (end -344.3732 128.6764) (width 0.3048) (layer "F.Cu") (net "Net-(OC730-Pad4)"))
 (segment (start -341.5303 125.5268) (end -341.5303 128.9201) (width 0.3048) (layer "F.Cu") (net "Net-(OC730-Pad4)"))
 (segment (start -353.9725 125.6284) (end -354.0252 125.6284) (width 0.3048) (layer "F.Cu") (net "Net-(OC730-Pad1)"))
 (segment (start -352.1983 128.8815) (end -351.9932 128.6764) (width 0.3048) (layer "F.Cu") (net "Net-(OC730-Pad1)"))
 (segment (start -355.092 126.6952) (end -355.092 128.8815) (width 0.3048) (layer "F.Cu") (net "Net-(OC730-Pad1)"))
 (segment (start -355.092 128.8815) (end -352.1983 128.8815) (width 0.3048) (layer "F.Cu") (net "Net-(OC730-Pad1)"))
 (segment (start -354.0252 125.6284) (end -355.092 126.6952) (width 0.3048) (layer "F.Cu") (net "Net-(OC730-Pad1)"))
 (segment (start -341.3252 135.128) (end -341.3252 136.398) (width 0.3048) (layer "F.Cu") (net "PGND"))
 (segment (start -343.7147 136.4507) (end -343.7636 136.4996) (width 0.3048) (layer "F.Cu") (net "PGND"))
 (segment (start -343.7147 134.9756) (end -343.5115 135.1788) (width 0.3048) (layer "F.Cu") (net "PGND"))
 (segment (start -343.5115 135.1788) (end -341.376 135.1788) (width 0.3048) (layer "F.Cu") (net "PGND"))
 (segment (start -341.376 135.1788) (end -341.3252 135.128) (width 0.3048) (layer "F.Cu") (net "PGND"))
 (segment (start -341.3252 136.398) (end -341.376 136.4488) (width 0.3048) (layer "F.Cu") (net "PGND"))
 (segment (start -343.7147 134.9756) (end -343.7147 136.4507) (width 0.3048) (layer "F.Cu") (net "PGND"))
 (via (at -346.6084 128.6002) (size 0.9144) (drill 0.4572) (layers "F.Cu" "B.Cu") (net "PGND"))
 (via (at -346.6338 131.6736) (size 0.9144) (drill 0.4572) (layers "F.Cu" "B.Cu") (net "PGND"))
 (via (at -339.2678 127.5334) (size 0.9144) (drill 0.4572) (layers "F.Cu" "B.Cu") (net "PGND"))
 (via (at -339.2678 131.0132) (size 0.9144) (drill 0.4572) (layers "F.Cu" "B.Cu") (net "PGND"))
 (via (at -347.98 123.8504) (size 1.4) (drill 0.7) (layers "F.Cu" "B.Cu") (tenting (front no) (back no)) (capping no)
  (covering (front no) (back no)) (plugging (front no) (back no)) (filling no) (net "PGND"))
 (via (at -343.7636 136.4996) (size 0.9144) (drill 0.4572) (layers "F.Cu" "B.Cu") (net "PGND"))
 (via (at -341.376 136.4488) (size 0.9144) (drill 0.4572) (layers "F.Cu" "B.Cu") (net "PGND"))
 (via (at -345.9988 125.8316) (size 0.9144) (drill 0.4572) (layers "F.Cu" "B.Cu") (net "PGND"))
 (via (at -347.98 134.874) (size 0.9144) (drill 0.4572) (layers "F.Cu" "B.Cu") (tenting (front no) (back no)) (capping no)
  (covering (front no) (back no)) (plugging (front no) (back no)) (filling no) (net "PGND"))
 (segment (start -347.98 135.9408) (end -347.98 123.8504) (width 0.3048) (layer "B.Cu") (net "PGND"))
 (segment (start -347.4212 136.4996) (end -347.98 135.9408) (width 0.3048) (layer "B.Cu") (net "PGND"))
 (segment (start -343.7636 136.4996) (end -347.4212 136.4996) (width 0.3048) (layer "B.Cu") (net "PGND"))
 (segment (start -338.5464 134.178) (end -337.9216 133.5532) (width 0.3048) (layer "F.Cu") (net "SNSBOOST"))
 (segment (start -339.450199 134.178) (end -338.5464 134.178) (width 0.3048) (layer "F.Cu") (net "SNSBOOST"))
 (segment (start -337.9216 133.5532) (end -337.9216 124.714) (width 0.3048) (layer "F.Cu") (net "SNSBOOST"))
 (segment (start -337.9216 124.714) (end -338.9376 123.698) (width 0.3048) (layer "F.Cu") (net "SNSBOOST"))
 (via (at -338.9376 123.698) (size 1.4) (drill 0.7) (layers "F.Cu" "B.Cu") (tenting (front no) (back no)) (capping no)
  (covering (front no) (back no)) (plugging (front no) (back no)) (filling no) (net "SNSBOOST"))
 (segment (start -352.0948 123.8504) (end -352.0948 125.5757) (width 0.3048) (layer "F.Cu") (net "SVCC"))
 (segment (start -352.0948 125.5757) (end -352.1475 125.6284) (width 0.3048) (layer "F.Cu") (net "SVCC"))
 (via (at -352.0948 123.8504) (size 1.4) (drill 0.7) (layers "F.Cu" "B.Cu") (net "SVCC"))
 (segment (start -343.3553 123.7507) (end -343.3572 123.7488) (width 0.3048) (layer "F.Cu") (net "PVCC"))
 (segment (start -343.3553 125.5268) (end -343.3553 123.7507) (width 0.3048) (layer "F.Cu") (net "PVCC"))
 (via (at -343.3572 123.7488) (size 1.4) (drill 0.7) (layers "F.Cu" "B.Cu") (tenting (front no) (back no)) (capping no)
  (covering (front no) (back no)) (plugging (front no) (back no)) (filling no) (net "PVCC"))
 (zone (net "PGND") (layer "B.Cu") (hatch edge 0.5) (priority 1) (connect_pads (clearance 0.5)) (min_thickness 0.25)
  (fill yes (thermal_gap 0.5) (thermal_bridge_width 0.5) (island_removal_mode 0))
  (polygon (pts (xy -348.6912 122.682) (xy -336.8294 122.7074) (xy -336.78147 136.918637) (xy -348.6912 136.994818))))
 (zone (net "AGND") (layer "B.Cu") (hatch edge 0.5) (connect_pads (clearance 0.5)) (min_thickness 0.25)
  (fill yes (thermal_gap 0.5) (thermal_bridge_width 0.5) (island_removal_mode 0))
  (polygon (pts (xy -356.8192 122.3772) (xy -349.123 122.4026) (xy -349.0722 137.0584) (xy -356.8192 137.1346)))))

